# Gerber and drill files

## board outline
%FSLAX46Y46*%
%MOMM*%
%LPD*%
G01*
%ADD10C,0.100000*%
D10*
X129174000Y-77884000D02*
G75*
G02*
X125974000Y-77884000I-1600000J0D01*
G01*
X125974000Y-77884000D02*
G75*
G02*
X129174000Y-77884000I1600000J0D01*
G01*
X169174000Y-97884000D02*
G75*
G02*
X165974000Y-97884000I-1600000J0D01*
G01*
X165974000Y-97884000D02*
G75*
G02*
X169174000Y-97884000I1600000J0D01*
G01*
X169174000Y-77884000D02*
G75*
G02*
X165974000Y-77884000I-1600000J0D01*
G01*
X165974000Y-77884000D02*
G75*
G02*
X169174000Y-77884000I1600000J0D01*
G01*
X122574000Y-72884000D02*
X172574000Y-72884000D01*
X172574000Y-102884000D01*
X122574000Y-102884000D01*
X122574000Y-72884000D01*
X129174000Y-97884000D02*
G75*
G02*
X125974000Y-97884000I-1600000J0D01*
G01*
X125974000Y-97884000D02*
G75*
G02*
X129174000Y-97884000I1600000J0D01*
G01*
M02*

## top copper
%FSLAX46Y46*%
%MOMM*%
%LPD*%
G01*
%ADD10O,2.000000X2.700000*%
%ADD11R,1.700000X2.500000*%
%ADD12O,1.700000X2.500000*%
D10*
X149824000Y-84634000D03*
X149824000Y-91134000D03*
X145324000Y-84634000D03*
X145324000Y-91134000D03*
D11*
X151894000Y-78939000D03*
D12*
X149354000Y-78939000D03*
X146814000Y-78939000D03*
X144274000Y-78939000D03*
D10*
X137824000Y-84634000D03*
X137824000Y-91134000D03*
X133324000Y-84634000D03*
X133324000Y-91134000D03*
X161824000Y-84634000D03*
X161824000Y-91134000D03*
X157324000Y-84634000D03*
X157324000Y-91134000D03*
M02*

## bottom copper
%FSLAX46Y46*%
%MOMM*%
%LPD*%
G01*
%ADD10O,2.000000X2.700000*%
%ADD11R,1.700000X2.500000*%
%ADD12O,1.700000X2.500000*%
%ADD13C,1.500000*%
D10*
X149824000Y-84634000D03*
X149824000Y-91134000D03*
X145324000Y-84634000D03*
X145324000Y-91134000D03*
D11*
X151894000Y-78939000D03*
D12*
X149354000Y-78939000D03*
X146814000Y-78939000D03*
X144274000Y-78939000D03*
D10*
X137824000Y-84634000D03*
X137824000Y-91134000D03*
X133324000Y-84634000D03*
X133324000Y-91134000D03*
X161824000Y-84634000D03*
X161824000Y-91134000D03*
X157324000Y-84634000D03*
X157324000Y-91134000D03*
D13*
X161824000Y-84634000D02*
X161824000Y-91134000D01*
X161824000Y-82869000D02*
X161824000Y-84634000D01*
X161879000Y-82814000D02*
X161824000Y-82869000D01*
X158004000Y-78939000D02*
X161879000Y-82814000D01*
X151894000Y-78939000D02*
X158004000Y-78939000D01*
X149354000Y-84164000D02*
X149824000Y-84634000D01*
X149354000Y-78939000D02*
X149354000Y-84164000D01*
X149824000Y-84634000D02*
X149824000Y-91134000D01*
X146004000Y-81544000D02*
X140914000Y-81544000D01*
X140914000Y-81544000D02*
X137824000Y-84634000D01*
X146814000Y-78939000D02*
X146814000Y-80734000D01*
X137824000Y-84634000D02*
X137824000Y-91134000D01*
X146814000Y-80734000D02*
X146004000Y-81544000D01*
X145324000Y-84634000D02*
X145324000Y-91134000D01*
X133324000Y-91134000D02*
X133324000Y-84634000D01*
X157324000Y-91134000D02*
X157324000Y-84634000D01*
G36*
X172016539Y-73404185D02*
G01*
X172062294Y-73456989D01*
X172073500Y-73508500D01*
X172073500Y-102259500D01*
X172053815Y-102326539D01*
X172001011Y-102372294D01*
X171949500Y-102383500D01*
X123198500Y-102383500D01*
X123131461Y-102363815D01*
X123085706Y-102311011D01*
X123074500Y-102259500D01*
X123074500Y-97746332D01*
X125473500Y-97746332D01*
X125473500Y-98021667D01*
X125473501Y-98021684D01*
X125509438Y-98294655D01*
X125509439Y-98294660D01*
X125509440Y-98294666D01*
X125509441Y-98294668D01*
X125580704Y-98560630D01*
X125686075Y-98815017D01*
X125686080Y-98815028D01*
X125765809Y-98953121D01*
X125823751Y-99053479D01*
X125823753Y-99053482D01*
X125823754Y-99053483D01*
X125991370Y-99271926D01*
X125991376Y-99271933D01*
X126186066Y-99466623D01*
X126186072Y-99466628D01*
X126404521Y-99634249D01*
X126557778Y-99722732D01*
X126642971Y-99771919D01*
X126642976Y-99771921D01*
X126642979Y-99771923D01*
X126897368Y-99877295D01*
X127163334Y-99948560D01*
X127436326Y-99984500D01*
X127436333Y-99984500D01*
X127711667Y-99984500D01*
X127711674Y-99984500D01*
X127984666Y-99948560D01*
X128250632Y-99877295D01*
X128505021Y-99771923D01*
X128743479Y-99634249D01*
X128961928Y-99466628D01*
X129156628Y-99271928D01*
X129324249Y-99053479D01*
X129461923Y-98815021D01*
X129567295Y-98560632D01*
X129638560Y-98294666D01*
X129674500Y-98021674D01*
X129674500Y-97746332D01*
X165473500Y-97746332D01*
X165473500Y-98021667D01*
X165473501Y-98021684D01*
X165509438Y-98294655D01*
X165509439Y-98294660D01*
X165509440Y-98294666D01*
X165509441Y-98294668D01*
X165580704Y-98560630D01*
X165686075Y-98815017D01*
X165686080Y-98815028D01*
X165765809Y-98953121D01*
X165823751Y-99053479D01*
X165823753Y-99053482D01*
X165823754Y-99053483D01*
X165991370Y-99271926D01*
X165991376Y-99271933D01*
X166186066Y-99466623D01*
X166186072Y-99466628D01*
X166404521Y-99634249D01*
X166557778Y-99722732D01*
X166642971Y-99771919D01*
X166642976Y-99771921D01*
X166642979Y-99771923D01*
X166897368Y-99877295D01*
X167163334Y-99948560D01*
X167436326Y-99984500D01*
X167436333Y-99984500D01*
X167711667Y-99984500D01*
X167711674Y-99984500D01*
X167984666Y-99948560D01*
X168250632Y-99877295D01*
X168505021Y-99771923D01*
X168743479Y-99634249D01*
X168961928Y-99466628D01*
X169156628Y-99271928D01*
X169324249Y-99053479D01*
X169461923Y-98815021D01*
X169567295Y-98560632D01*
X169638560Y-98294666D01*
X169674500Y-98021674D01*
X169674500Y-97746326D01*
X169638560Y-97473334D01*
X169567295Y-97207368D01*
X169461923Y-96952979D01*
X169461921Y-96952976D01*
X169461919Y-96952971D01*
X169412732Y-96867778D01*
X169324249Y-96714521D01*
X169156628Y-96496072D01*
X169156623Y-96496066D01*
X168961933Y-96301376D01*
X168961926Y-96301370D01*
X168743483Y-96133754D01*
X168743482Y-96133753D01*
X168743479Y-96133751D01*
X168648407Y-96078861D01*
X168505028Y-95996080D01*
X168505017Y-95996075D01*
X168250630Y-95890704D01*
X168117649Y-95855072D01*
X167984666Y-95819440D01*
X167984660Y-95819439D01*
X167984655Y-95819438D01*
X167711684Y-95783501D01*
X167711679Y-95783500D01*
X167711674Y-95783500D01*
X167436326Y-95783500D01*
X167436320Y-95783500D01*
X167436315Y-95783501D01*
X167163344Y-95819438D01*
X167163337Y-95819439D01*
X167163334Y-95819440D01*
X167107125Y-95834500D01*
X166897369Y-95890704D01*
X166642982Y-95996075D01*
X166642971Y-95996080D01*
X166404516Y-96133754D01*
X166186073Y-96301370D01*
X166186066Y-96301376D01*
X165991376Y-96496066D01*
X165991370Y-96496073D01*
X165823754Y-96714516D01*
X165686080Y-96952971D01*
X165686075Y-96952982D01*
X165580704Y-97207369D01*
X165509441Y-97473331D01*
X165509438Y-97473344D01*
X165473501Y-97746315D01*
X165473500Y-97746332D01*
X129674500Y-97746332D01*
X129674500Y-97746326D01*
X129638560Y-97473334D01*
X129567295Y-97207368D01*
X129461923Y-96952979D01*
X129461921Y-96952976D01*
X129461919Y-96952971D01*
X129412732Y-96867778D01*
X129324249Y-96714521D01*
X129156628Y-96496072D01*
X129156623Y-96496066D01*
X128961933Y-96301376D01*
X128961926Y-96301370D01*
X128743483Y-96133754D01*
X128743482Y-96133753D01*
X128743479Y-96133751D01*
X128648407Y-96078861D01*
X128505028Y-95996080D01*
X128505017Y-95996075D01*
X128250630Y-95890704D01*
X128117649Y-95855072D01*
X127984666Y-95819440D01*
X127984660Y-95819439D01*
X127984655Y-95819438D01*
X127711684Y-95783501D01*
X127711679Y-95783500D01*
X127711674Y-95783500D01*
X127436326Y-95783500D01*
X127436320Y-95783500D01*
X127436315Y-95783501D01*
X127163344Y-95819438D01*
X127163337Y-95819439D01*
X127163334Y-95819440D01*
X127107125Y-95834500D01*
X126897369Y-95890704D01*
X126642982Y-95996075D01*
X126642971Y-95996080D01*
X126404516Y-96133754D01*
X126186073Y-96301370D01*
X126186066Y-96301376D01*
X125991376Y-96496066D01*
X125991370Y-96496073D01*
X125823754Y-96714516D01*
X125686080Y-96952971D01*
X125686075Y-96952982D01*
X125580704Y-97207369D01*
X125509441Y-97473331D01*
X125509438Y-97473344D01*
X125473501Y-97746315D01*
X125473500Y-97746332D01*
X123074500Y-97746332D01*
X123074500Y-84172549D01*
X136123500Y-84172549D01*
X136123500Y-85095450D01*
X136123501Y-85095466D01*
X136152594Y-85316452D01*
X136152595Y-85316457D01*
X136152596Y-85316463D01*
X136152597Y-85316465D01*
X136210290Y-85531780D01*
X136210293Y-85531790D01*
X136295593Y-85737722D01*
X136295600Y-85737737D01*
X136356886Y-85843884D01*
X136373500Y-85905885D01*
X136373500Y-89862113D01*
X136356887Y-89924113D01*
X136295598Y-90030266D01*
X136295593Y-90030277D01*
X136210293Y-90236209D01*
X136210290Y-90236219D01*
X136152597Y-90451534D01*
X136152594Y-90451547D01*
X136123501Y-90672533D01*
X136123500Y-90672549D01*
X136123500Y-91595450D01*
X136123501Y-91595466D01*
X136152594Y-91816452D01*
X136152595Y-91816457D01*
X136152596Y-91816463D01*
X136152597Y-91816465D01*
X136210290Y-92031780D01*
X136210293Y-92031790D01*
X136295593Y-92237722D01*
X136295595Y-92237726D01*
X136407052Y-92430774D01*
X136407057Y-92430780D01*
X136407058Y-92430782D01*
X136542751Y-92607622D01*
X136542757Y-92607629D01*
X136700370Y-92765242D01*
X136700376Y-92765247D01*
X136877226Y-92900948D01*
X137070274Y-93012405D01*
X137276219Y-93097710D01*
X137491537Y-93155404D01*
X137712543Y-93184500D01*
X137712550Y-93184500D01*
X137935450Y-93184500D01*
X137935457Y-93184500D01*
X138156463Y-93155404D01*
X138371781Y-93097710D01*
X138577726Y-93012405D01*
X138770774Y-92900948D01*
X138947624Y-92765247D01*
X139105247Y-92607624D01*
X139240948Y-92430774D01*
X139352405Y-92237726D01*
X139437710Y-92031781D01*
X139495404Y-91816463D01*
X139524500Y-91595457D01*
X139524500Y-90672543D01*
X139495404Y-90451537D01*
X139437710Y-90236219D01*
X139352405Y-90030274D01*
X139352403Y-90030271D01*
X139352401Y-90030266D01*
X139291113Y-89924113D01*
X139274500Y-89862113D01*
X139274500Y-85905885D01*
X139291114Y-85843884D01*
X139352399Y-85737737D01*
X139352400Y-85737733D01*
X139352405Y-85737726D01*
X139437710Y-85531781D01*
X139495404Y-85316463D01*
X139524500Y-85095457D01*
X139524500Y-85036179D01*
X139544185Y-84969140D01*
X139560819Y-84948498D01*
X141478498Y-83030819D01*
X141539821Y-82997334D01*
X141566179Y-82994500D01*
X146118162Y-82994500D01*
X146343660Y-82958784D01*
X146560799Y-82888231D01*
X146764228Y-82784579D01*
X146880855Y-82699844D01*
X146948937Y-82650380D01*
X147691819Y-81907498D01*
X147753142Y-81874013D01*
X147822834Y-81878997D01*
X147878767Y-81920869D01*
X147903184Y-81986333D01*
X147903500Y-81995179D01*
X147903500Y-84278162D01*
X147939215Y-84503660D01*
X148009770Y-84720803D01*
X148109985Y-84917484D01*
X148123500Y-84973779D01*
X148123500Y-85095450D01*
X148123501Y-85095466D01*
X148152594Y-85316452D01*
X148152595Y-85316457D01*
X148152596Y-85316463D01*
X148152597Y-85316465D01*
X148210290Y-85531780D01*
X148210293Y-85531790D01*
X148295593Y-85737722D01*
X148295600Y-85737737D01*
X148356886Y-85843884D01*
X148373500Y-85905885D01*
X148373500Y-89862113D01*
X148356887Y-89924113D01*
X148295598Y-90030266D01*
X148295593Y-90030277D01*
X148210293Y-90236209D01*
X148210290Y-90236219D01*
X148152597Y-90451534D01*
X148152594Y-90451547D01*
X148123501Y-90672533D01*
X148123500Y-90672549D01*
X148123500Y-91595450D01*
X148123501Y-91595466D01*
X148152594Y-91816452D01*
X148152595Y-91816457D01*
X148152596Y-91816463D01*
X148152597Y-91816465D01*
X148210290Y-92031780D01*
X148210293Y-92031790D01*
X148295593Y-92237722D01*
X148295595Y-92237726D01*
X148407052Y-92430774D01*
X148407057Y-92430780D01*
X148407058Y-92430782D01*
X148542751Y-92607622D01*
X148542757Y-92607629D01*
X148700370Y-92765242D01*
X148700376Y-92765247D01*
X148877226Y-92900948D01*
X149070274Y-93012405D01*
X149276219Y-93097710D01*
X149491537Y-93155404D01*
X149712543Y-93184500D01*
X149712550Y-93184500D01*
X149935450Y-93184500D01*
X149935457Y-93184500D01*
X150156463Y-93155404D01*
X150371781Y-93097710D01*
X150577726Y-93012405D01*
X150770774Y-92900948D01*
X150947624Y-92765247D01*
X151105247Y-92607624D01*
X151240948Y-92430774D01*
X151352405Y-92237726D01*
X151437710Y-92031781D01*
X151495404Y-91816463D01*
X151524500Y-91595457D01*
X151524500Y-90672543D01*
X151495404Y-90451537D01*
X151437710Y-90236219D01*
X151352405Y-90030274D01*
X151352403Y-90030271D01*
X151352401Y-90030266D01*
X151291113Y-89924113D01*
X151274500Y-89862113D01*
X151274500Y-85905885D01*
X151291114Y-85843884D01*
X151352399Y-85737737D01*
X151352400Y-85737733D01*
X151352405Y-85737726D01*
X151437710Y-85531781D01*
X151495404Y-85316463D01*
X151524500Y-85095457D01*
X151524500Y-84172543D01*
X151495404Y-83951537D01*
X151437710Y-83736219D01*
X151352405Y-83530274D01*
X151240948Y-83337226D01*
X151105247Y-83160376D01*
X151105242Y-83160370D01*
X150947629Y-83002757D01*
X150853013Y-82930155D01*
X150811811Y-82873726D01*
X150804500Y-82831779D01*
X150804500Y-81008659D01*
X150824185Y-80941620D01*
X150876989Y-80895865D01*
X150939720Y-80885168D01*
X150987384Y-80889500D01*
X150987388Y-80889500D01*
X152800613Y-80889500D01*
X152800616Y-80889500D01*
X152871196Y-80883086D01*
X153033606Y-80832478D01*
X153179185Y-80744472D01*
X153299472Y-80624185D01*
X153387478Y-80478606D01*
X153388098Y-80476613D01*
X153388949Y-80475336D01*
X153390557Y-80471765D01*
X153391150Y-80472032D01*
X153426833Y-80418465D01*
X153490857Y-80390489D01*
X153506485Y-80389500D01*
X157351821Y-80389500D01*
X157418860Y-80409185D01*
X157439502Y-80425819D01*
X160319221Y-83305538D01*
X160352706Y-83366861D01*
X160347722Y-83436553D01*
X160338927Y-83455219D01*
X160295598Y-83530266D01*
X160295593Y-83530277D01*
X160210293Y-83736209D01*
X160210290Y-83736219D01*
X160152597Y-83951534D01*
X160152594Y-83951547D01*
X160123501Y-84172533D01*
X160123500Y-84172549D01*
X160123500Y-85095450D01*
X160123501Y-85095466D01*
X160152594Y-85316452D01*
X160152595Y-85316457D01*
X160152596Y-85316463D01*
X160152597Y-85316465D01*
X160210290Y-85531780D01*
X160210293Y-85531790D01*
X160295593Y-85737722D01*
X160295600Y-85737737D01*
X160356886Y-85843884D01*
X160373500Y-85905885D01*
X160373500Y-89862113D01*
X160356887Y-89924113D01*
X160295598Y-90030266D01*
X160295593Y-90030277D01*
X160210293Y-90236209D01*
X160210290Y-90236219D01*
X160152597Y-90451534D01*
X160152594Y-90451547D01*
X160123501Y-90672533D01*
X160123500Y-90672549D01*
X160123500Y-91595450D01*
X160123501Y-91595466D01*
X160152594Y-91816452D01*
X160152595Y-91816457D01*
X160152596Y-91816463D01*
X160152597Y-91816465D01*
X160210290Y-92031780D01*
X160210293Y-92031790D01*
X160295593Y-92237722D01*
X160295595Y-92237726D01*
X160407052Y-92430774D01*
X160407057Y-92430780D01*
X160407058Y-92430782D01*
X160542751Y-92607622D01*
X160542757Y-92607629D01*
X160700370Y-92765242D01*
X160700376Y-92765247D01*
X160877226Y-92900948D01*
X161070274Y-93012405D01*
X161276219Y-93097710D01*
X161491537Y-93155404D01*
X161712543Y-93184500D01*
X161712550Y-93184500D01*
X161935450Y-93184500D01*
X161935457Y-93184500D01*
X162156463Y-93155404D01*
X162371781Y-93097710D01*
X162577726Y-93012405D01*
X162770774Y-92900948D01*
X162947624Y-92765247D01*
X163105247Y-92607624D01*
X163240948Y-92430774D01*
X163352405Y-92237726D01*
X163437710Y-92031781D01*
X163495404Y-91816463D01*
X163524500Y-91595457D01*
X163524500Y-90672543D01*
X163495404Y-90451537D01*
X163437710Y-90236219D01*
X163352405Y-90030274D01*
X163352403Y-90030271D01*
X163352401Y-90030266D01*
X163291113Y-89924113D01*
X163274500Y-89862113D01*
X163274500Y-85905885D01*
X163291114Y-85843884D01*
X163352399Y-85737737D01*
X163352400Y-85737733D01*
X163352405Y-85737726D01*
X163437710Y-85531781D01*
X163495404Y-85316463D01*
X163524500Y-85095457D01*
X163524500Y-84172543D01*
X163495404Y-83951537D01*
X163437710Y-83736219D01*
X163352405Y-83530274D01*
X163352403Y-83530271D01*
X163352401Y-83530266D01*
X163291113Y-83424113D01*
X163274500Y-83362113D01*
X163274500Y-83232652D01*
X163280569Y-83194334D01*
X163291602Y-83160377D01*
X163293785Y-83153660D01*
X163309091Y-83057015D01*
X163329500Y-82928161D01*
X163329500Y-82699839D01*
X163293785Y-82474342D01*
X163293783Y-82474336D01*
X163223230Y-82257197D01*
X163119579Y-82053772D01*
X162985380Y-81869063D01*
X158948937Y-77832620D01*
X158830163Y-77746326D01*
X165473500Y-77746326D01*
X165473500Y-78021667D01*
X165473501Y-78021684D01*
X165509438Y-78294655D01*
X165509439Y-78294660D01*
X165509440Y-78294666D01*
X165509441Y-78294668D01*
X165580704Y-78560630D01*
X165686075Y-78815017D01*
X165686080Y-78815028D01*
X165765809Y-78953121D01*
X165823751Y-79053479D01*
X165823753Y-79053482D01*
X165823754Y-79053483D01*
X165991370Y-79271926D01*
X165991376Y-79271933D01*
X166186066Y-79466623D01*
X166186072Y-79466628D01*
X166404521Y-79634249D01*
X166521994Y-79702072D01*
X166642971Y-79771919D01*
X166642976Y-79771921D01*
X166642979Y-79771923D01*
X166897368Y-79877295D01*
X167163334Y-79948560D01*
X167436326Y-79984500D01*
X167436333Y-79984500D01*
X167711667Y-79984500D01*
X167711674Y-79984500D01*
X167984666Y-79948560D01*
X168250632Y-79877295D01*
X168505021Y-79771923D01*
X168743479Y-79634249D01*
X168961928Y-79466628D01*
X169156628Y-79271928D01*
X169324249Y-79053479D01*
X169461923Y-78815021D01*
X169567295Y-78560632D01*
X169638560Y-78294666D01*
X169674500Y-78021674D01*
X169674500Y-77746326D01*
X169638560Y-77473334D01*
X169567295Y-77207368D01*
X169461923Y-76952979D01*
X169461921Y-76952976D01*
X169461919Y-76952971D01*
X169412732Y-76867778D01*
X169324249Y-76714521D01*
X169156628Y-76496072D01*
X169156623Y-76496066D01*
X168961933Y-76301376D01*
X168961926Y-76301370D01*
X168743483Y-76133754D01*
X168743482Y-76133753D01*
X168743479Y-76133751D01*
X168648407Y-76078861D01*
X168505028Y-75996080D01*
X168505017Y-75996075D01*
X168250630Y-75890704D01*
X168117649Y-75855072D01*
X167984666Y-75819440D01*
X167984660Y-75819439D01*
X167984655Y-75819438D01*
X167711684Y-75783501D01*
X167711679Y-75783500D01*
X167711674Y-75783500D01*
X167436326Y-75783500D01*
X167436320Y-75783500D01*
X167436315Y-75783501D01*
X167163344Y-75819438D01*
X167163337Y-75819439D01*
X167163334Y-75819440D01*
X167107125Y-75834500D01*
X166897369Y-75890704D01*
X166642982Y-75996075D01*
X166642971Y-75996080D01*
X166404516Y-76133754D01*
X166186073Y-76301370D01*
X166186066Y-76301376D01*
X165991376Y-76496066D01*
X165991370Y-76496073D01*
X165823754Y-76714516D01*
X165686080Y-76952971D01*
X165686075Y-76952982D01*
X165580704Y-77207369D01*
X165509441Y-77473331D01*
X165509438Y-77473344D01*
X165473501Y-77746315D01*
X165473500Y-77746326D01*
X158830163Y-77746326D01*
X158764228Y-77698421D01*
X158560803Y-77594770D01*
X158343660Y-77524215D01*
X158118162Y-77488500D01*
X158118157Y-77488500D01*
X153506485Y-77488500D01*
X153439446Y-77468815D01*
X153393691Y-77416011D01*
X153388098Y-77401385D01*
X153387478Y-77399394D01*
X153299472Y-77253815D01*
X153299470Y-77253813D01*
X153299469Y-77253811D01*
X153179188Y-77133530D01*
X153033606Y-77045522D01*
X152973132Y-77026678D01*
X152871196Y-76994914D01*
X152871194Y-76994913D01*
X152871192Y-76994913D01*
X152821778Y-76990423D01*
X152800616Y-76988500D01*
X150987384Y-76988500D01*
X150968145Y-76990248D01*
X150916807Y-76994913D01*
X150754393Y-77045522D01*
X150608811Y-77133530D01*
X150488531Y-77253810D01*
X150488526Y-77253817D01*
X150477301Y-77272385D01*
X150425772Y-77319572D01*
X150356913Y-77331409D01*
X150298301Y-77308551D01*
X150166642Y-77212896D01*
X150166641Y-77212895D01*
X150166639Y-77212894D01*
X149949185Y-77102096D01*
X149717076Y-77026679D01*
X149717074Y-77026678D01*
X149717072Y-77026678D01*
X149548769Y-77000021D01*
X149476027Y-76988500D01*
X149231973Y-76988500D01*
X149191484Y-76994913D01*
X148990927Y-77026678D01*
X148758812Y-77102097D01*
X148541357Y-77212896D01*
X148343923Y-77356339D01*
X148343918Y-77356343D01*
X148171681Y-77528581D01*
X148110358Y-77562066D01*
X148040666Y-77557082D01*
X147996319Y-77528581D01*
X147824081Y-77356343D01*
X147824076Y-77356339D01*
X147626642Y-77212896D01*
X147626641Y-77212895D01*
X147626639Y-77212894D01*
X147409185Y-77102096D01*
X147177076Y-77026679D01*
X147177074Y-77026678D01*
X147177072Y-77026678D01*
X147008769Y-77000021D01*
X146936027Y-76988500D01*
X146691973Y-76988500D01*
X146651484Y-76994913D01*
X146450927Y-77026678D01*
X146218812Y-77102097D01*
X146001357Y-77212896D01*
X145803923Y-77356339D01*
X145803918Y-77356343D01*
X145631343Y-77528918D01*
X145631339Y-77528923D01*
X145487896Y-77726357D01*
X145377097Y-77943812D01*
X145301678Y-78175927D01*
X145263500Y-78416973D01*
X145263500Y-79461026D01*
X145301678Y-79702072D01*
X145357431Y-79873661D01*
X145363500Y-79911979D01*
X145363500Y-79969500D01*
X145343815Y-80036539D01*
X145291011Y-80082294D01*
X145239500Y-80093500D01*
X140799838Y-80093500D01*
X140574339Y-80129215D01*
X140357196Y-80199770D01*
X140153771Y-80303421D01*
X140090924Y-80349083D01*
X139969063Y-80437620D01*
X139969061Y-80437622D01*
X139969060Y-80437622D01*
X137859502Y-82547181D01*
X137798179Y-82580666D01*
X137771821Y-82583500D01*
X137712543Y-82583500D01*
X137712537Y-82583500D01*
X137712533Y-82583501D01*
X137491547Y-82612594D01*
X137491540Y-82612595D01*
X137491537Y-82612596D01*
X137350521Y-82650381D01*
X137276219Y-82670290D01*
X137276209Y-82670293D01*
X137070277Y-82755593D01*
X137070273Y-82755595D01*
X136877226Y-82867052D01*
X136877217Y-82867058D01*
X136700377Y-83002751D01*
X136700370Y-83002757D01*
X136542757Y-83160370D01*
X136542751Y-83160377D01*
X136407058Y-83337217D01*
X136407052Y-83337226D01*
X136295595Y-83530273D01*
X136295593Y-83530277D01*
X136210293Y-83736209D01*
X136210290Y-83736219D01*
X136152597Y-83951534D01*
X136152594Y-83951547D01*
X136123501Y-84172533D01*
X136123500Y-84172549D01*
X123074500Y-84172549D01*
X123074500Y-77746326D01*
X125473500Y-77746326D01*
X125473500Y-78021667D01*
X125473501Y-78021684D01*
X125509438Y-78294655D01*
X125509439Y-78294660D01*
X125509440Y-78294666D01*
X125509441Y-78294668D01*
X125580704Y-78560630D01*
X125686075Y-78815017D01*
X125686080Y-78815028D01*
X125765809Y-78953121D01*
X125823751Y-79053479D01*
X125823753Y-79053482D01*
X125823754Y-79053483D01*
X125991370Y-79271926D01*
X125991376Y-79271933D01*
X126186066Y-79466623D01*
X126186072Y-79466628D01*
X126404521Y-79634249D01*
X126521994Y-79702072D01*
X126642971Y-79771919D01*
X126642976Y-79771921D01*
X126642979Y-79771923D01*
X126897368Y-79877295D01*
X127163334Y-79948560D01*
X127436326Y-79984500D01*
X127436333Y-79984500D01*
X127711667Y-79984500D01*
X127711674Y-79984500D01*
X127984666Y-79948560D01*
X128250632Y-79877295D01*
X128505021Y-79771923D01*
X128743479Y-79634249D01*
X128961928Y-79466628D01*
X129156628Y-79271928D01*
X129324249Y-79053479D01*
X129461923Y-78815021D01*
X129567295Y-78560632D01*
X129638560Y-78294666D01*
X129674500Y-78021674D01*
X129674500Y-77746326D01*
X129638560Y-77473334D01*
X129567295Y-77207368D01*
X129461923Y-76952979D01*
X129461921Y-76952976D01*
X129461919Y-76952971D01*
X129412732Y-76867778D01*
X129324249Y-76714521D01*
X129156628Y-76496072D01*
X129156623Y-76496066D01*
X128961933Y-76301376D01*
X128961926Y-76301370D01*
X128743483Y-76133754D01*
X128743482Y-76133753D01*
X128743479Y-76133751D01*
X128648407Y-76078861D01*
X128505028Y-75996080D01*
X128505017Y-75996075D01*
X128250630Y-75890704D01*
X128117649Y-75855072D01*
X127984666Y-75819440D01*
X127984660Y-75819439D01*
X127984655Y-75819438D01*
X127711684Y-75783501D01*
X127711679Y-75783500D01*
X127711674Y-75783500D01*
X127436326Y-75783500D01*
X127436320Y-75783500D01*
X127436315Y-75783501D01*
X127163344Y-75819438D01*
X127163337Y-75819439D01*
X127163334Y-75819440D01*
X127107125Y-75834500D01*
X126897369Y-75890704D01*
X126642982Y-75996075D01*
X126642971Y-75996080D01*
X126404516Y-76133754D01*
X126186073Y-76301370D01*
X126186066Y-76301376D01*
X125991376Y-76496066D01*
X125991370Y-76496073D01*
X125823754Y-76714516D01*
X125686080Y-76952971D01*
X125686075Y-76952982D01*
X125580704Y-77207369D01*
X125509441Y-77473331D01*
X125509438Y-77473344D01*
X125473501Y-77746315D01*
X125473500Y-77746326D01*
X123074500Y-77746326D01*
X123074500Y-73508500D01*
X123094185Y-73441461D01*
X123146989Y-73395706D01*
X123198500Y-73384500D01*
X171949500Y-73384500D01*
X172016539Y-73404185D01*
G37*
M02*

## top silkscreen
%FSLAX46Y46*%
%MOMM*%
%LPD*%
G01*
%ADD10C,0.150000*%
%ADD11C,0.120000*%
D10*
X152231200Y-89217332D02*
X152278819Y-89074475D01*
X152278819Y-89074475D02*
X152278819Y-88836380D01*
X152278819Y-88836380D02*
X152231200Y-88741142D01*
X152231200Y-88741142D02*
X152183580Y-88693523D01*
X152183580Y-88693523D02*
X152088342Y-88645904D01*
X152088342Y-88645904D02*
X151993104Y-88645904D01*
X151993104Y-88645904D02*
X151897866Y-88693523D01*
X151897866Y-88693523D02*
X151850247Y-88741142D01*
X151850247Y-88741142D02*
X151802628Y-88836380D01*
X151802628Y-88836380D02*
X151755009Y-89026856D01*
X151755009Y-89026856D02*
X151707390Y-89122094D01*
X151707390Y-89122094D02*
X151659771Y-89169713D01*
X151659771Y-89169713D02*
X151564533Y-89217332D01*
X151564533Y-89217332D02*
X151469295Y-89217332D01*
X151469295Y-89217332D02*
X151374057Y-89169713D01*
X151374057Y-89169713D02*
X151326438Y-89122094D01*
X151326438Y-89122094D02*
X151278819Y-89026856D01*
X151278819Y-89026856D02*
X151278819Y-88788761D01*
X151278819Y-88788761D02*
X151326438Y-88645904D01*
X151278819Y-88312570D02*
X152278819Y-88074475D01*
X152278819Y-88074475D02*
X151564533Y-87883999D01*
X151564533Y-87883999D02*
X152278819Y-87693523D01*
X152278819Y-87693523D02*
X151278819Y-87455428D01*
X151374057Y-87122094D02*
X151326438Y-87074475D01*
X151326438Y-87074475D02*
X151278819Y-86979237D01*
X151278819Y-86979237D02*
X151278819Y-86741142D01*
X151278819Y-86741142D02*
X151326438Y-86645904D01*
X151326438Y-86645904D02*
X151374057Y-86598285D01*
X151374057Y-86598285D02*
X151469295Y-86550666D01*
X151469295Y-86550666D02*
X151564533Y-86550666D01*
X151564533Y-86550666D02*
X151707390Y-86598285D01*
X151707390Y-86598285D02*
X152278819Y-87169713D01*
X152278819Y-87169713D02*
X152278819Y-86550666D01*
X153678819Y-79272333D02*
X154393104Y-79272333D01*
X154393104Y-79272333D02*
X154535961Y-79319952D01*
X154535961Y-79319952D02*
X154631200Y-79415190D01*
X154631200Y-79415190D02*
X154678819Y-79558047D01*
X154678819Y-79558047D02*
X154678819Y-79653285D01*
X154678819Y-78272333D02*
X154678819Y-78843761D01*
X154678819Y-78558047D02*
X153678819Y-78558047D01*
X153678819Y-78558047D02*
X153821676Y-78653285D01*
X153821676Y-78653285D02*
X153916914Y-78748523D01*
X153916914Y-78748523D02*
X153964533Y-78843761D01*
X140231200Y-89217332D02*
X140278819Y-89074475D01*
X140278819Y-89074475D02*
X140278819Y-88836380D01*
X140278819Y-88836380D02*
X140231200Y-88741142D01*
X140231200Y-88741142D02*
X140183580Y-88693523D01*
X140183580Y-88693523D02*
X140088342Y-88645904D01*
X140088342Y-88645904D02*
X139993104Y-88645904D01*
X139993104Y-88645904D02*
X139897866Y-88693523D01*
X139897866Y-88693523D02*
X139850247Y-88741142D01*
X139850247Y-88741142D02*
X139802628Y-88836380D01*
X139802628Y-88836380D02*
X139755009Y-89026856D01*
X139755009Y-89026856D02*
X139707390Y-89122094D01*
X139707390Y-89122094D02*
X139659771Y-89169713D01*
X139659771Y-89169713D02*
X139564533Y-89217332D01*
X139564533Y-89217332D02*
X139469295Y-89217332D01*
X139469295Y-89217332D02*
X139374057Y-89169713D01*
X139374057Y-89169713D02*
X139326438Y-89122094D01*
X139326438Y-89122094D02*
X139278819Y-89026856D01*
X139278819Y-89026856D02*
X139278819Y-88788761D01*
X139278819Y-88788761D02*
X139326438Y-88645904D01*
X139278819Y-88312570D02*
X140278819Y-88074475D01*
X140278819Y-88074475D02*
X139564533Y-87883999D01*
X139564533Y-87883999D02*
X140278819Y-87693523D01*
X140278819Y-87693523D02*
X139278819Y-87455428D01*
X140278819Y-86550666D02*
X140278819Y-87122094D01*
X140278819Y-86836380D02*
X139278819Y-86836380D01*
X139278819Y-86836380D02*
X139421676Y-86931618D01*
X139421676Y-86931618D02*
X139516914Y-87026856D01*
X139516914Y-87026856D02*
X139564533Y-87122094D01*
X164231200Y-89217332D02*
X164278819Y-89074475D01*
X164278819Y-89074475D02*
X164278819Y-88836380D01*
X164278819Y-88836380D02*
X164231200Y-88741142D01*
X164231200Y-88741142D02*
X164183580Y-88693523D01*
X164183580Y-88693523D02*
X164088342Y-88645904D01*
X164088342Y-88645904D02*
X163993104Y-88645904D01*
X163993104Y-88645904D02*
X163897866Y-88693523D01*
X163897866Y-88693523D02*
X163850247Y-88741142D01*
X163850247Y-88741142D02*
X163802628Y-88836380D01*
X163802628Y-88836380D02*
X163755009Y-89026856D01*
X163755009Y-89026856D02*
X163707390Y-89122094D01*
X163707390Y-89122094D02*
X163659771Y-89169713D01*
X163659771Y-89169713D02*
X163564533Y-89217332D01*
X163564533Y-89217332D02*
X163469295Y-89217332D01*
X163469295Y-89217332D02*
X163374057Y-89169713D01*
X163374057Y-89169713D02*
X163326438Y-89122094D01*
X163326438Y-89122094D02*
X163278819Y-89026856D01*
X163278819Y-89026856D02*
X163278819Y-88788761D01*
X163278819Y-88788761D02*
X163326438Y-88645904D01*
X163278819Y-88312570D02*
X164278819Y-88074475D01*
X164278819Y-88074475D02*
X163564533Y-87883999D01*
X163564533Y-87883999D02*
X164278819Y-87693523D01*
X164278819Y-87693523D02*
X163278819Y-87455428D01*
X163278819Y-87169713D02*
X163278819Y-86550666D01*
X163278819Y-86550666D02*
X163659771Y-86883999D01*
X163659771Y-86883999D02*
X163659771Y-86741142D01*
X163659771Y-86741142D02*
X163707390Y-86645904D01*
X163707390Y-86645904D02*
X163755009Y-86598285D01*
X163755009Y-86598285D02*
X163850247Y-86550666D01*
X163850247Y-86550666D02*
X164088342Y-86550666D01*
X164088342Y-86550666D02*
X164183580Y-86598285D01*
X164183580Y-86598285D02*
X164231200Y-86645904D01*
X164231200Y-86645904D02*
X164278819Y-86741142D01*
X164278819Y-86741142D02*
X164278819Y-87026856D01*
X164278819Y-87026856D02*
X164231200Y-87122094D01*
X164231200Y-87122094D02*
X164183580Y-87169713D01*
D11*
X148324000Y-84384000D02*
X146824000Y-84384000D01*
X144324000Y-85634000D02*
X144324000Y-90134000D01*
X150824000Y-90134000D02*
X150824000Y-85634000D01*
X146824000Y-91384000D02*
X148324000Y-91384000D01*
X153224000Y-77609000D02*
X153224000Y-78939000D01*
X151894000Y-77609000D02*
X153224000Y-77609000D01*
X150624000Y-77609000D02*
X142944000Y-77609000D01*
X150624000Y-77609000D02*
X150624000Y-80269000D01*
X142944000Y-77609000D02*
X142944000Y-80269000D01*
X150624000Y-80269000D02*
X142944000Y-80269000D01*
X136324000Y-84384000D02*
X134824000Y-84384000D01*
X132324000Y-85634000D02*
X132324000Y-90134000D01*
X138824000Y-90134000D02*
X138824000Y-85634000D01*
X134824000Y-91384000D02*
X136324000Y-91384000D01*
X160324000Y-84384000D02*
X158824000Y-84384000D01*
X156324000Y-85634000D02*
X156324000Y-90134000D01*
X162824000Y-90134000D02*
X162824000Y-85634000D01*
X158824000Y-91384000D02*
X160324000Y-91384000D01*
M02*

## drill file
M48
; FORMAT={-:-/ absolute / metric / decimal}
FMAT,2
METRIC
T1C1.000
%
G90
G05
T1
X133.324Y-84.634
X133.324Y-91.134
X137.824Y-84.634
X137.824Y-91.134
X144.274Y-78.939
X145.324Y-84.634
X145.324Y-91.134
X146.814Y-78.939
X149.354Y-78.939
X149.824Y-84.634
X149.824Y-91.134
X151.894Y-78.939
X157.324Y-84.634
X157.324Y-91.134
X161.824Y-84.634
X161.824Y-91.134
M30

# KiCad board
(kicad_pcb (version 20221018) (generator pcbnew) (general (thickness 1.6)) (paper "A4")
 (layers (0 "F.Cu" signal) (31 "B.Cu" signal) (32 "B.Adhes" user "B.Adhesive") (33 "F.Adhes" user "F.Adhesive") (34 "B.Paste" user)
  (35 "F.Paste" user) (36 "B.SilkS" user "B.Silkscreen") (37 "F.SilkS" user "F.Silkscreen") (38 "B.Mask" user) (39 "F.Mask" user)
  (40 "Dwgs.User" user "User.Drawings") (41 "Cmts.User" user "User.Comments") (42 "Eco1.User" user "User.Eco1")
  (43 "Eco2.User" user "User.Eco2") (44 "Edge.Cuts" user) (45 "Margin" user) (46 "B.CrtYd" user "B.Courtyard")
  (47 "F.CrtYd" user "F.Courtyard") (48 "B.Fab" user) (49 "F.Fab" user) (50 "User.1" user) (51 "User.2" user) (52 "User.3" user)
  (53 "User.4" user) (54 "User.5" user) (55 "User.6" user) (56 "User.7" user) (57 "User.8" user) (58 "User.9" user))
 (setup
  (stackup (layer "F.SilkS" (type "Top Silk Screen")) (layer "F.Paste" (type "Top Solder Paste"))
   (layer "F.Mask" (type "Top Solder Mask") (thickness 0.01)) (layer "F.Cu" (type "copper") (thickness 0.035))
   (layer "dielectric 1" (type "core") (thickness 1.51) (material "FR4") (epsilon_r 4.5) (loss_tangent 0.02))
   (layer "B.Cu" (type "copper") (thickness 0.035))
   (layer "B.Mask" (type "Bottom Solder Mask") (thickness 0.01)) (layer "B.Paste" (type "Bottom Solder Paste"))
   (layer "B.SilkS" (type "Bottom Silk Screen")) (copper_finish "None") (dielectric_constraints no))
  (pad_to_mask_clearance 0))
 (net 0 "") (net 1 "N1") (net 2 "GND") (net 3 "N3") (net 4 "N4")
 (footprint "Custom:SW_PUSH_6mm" (layer "F.Cu") (at 149.824 84.634 -90)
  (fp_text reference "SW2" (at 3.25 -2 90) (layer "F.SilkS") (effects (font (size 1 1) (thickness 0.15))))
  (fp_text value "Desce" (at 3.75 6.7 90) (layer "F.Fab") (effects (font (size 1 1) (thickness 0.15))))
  (fp_line (start -0.25 1.5) (end -0.25 3) (stroke (width 0.12) (type solid)) (layer "F.SilkS"))
  (fp_line (start 1 5.5) (end 5.5 5.5) (stroke (width 0.12) (type solid)) (layer "F.SilkS"))
  (fp_line (start 5.5 -1) (end 1 -1) (stroke (width 0.12) (type solid)) (layer "F.SilkS"))
  (fp_line (start 6.75 3) (end 6.75 1.5) (stroke (width 0.12) (type solid)) (layer "F.SilkS"))
  (pad "1" thru_hole oval (at 0 0) (size 2 2.7) (drill 1) (layers "*.Cu" "*.Mask") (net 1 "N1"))
  (pad "1" thru_hole oval (at 6.5 0) (size 2 2.7) (drill 1) (layers "*.Cu" "*.Mask") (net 1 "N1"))
  (pad "2" thru_hole oval (at 0 4.5) (size 2 2.7) (drill 1) (layers "*.Cu" "*.Mask") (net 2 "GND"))
  (pad "2" thru_hole oval (at 6.5 4.5) (size 2 2.7) (drill 1) (layers "*.Cu" "*.Mask") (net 2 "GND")))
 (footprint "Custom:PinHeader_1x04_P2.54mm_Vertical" (layer "F.Cu") (at 151.894 78.939 -90)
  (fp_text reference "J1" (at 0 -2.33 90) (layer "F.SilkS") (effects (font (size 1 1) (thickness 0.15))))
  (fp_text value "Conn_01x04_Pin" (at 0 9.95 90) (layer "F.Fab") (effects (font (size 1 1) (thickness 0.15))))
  (fp_line (start -1.33 -1.33) (end 0 -1.33) (stroke (width 0.12) (type solid)) (layer "F.SilkS"))
  (fp_line (start -1.33 0) (end -1.33 -1.33) (stroke (width 0.12) (type solid)) (layer "F.SilkS"))
  (fp_line (start -1.33 1.27) (end -1.33 8.95) (stroke (width 0.12) (type solid)) (layer "F.SilkS"))
  (fp_line (start -1.33 1.27) (end 1.33 1.27) (stroke (width 0.12) (type solid)) (layer "F.SilkS"))
  (fp_line (start -1.33 8.95) (end 1.33 8.95) (stroke (width 0.12) (type solid)) (layer "F.SilkS"))
  (fp_line (start 1.33 1.27) (end 1.33 8.95) (stroke (width 0.12) (type solid)) (layer "F.SilkS"))
  (pad "1" thru_hole rect (at 0 0 270) (size 2.5 1.7) (drill 1) (layers "*.Cu" "*.Mask") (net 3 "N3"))
  (pad "2" thru_hole oval (at 0 2.54 270) (size 2.5 1.7) (drill 1) (layers "*.Cu" "*.Mask") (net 1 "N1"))
  (pad "3" thru_hole oval (at 0 5.08 270) (size 2.5 1.7) (drill 1) (layers "*.Cu" "*.Mask") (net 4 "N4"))
  (pad "4" thru_hole oval (at 0 7.62 270) (size 2.5 1.7) (drill 1) (layers "*.Cu" "*.Mask") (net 2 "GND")))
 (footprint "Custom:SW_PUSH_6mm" (layer "F.Cu") (at 137.824 84.634 -90)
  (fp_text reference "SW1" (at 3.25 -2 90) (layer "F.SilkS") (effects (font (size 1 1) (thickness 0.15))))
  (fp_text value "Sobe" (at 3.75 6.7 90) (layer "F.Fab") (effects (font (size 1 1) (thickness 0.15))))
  (fp_line (start -0.25 1.5) (end -0.25 3) (stroke (width 0.12) (type solid)) (layer "F.SilkS"))
  (fp_line (start 1 5.5) (end 5.5 5.5) (stroke (width 0.12) (type solid)) (layer "F.SilkS"))
  (fp_line (start 5.5 -1) (end 1 -1) (stroke (width 0.12) (type solid)) (layer "F.SilkS"))
  (fp_line (start 6.75 3) (end 6.75 1.5) (stroke (width 0.12) (type solid)) (layer "F.SilkS"))
  (pad "1" thru_hole oval (at 0 0) (size 2 2.7) (drill 1) (layers "*.Cu" "*.Mask") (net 4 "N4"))
  (pad "1" thru_hole oval (at 6.5 0) (size 2 2.7) (drill 1) (layers "*.Cu" "*.Mask") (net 4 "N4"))
  (pad "2" thru_hole oval (at 0 4.5) (size 2 2.7) (drill 1) (layers "*.Cu" "*.Mask") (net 2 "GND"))
  (pad "2" thru_hole oval (at 6.5 4.5) (size 2 2.7) (drill 1) (layers "*.Cu" "*.Mask") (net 2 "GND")))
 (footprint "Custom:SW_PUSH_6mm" (layer "F.Cu") (at 161.824 84.634 -90)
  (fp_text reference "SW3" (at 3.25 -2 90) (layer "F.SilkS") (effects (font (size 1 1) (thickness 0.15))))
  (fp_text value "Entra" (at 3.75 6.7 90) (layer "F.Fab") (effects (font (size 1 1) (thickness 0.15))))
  (fp_line (start -0.25 1.5) (end -0.25 3) (stroke (width 0.12) (type solid)) (layer "F.SilkS"))
  (fp_line (start 1 5.5) (end 5.5 5.5) (stroke (width 0.12) (type solid)) (layer "F.SilkS"))
  (fp_line (start 5.5 -1) (end 1 -1) (stroke (width 0.12) (type solid)) (layer "F.SilkS"))
  (fp_line (start 6.75 3) (end 6.75 1.5) (stroke (width 0.12) (type solid)) (layer "F.SilkS"))
  (pad "1" thru_hole oval (at 0 0) (size 2 2.7) (drill 1) (layers "*.Cu" "*.Mask") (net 3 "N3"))
  (pad "1" thru_hole oval (at 6.5 0) (size 2 2.7) (drill 1) (layers "*.Cu" "*.Mask") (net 3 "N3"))
  (pad "2" thru_hole oval (at 0 4.5) (size 2 2.7) (drill 1) (layers "*.Cu" "*.Mask") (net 2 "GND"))
  (pad "2" thru_hole oval (at 6.5 4.5) (size 2 2.7) (drill 1) (layers "*.Cu" "*.Mask") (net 2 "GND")))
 (gr_circle (center 127.574 77.884) (end 129.174 77.884) (stroke (width 0.1) (type default)) (fill none) (layer "Edge.Cuts"))
 (gr_circle (center 167.574 97.884) (end 169.174 97.884) (stroke (width 0.1) (type default)) (fill none) (layer "Edge.Cuts"))
 (gr_circle (center 167.574 77.884) (end 169.174 77.884) (stroke (width 0.1) (type default)) (fill none) (layer "Edge.Cuts"))
 (gr_rect (start 122.574 72.884) (end 172.574 102.884) (stroke (width 0.1) (type default)) (fill none) (layer "Edge.Cuts"))
 (gr_circle (center 127.574 97.884) (end 129.174 97.884) (stroke (width 0.1) (type default)) (fill none) (layer "Edge.Cuts"))
 (segment (start 161.824 84.634) (end 161.824 91.134) (width 1.5) (layer "B.Cu") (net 3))
 (segment (start 161.824 82.869) (end 161.824 84.634) (width 1.5) (layer "B.Cu") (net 3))
 (segment (start 161.879 82.814) (end 161.824 82.869) (width 1.5) (layer "B.Cu") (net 3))
 (segment (start 158.004 78.939) (end 161.879 82.814) (width 1.5) (layer "B.Cu") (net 3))
 (segment (start 151.894 78.939) (end 158.004 78.939) (width 1.5) (layer "B.Cu") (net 3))
 (segment (start 149.354 84.164) (end 149.824 84.634) (width 1.5) (layer "B.Cu") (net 1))
 (segment (start 149.354 78.939) (end 149.354 84.164) (width 1.5) (layer "B.Cu") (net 1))
 (segment (start 149.824 84.634) (end 149.824 91.134) (width 1.5) (layer "B.Cu") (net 1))
 (segment (start 146.004 81.544) (end 140.914 81.544) (width 1.5) (layer "B.Cu") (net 4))
 (segment (start 140.914 81.544) (end 137.824 84.634) (width 1.5) (layer "B.Cu") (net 4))
 (segment (start 146.814 78.939) (end 146.814 80.734) (width 1.5) (layer "B.Cu") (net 4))
 (segment (start 137.824 84.634) (end 137.824 91.134) (width 1.5) (layer "B.Cu") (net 4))
 (segment (start 146.814 80.734) (end 146.004 81.544) (width 1.5) (layer "B.Cu") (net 4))
 (segment (start 145.324 84.634) (end 145.324 91.134) (width 1.5) (layer "B.Cu") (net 2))
 (segment (start 133.324 91.134) (end 133.324 84.634) (width 1.5) (layer "B.Cu") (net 2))
 (segment (start 157.324 91.134) (end 157.324 84.634) (width 1.5) (layer "B.Cu") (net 2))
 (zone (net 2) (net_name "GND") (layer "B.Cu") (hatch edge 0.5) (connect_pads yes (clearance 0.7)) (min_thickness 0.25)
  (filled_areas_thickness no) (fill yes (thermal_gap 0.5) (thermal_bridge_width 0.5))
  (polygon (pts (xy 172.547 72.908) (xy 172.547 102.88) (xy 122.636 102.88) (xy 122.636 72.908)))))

